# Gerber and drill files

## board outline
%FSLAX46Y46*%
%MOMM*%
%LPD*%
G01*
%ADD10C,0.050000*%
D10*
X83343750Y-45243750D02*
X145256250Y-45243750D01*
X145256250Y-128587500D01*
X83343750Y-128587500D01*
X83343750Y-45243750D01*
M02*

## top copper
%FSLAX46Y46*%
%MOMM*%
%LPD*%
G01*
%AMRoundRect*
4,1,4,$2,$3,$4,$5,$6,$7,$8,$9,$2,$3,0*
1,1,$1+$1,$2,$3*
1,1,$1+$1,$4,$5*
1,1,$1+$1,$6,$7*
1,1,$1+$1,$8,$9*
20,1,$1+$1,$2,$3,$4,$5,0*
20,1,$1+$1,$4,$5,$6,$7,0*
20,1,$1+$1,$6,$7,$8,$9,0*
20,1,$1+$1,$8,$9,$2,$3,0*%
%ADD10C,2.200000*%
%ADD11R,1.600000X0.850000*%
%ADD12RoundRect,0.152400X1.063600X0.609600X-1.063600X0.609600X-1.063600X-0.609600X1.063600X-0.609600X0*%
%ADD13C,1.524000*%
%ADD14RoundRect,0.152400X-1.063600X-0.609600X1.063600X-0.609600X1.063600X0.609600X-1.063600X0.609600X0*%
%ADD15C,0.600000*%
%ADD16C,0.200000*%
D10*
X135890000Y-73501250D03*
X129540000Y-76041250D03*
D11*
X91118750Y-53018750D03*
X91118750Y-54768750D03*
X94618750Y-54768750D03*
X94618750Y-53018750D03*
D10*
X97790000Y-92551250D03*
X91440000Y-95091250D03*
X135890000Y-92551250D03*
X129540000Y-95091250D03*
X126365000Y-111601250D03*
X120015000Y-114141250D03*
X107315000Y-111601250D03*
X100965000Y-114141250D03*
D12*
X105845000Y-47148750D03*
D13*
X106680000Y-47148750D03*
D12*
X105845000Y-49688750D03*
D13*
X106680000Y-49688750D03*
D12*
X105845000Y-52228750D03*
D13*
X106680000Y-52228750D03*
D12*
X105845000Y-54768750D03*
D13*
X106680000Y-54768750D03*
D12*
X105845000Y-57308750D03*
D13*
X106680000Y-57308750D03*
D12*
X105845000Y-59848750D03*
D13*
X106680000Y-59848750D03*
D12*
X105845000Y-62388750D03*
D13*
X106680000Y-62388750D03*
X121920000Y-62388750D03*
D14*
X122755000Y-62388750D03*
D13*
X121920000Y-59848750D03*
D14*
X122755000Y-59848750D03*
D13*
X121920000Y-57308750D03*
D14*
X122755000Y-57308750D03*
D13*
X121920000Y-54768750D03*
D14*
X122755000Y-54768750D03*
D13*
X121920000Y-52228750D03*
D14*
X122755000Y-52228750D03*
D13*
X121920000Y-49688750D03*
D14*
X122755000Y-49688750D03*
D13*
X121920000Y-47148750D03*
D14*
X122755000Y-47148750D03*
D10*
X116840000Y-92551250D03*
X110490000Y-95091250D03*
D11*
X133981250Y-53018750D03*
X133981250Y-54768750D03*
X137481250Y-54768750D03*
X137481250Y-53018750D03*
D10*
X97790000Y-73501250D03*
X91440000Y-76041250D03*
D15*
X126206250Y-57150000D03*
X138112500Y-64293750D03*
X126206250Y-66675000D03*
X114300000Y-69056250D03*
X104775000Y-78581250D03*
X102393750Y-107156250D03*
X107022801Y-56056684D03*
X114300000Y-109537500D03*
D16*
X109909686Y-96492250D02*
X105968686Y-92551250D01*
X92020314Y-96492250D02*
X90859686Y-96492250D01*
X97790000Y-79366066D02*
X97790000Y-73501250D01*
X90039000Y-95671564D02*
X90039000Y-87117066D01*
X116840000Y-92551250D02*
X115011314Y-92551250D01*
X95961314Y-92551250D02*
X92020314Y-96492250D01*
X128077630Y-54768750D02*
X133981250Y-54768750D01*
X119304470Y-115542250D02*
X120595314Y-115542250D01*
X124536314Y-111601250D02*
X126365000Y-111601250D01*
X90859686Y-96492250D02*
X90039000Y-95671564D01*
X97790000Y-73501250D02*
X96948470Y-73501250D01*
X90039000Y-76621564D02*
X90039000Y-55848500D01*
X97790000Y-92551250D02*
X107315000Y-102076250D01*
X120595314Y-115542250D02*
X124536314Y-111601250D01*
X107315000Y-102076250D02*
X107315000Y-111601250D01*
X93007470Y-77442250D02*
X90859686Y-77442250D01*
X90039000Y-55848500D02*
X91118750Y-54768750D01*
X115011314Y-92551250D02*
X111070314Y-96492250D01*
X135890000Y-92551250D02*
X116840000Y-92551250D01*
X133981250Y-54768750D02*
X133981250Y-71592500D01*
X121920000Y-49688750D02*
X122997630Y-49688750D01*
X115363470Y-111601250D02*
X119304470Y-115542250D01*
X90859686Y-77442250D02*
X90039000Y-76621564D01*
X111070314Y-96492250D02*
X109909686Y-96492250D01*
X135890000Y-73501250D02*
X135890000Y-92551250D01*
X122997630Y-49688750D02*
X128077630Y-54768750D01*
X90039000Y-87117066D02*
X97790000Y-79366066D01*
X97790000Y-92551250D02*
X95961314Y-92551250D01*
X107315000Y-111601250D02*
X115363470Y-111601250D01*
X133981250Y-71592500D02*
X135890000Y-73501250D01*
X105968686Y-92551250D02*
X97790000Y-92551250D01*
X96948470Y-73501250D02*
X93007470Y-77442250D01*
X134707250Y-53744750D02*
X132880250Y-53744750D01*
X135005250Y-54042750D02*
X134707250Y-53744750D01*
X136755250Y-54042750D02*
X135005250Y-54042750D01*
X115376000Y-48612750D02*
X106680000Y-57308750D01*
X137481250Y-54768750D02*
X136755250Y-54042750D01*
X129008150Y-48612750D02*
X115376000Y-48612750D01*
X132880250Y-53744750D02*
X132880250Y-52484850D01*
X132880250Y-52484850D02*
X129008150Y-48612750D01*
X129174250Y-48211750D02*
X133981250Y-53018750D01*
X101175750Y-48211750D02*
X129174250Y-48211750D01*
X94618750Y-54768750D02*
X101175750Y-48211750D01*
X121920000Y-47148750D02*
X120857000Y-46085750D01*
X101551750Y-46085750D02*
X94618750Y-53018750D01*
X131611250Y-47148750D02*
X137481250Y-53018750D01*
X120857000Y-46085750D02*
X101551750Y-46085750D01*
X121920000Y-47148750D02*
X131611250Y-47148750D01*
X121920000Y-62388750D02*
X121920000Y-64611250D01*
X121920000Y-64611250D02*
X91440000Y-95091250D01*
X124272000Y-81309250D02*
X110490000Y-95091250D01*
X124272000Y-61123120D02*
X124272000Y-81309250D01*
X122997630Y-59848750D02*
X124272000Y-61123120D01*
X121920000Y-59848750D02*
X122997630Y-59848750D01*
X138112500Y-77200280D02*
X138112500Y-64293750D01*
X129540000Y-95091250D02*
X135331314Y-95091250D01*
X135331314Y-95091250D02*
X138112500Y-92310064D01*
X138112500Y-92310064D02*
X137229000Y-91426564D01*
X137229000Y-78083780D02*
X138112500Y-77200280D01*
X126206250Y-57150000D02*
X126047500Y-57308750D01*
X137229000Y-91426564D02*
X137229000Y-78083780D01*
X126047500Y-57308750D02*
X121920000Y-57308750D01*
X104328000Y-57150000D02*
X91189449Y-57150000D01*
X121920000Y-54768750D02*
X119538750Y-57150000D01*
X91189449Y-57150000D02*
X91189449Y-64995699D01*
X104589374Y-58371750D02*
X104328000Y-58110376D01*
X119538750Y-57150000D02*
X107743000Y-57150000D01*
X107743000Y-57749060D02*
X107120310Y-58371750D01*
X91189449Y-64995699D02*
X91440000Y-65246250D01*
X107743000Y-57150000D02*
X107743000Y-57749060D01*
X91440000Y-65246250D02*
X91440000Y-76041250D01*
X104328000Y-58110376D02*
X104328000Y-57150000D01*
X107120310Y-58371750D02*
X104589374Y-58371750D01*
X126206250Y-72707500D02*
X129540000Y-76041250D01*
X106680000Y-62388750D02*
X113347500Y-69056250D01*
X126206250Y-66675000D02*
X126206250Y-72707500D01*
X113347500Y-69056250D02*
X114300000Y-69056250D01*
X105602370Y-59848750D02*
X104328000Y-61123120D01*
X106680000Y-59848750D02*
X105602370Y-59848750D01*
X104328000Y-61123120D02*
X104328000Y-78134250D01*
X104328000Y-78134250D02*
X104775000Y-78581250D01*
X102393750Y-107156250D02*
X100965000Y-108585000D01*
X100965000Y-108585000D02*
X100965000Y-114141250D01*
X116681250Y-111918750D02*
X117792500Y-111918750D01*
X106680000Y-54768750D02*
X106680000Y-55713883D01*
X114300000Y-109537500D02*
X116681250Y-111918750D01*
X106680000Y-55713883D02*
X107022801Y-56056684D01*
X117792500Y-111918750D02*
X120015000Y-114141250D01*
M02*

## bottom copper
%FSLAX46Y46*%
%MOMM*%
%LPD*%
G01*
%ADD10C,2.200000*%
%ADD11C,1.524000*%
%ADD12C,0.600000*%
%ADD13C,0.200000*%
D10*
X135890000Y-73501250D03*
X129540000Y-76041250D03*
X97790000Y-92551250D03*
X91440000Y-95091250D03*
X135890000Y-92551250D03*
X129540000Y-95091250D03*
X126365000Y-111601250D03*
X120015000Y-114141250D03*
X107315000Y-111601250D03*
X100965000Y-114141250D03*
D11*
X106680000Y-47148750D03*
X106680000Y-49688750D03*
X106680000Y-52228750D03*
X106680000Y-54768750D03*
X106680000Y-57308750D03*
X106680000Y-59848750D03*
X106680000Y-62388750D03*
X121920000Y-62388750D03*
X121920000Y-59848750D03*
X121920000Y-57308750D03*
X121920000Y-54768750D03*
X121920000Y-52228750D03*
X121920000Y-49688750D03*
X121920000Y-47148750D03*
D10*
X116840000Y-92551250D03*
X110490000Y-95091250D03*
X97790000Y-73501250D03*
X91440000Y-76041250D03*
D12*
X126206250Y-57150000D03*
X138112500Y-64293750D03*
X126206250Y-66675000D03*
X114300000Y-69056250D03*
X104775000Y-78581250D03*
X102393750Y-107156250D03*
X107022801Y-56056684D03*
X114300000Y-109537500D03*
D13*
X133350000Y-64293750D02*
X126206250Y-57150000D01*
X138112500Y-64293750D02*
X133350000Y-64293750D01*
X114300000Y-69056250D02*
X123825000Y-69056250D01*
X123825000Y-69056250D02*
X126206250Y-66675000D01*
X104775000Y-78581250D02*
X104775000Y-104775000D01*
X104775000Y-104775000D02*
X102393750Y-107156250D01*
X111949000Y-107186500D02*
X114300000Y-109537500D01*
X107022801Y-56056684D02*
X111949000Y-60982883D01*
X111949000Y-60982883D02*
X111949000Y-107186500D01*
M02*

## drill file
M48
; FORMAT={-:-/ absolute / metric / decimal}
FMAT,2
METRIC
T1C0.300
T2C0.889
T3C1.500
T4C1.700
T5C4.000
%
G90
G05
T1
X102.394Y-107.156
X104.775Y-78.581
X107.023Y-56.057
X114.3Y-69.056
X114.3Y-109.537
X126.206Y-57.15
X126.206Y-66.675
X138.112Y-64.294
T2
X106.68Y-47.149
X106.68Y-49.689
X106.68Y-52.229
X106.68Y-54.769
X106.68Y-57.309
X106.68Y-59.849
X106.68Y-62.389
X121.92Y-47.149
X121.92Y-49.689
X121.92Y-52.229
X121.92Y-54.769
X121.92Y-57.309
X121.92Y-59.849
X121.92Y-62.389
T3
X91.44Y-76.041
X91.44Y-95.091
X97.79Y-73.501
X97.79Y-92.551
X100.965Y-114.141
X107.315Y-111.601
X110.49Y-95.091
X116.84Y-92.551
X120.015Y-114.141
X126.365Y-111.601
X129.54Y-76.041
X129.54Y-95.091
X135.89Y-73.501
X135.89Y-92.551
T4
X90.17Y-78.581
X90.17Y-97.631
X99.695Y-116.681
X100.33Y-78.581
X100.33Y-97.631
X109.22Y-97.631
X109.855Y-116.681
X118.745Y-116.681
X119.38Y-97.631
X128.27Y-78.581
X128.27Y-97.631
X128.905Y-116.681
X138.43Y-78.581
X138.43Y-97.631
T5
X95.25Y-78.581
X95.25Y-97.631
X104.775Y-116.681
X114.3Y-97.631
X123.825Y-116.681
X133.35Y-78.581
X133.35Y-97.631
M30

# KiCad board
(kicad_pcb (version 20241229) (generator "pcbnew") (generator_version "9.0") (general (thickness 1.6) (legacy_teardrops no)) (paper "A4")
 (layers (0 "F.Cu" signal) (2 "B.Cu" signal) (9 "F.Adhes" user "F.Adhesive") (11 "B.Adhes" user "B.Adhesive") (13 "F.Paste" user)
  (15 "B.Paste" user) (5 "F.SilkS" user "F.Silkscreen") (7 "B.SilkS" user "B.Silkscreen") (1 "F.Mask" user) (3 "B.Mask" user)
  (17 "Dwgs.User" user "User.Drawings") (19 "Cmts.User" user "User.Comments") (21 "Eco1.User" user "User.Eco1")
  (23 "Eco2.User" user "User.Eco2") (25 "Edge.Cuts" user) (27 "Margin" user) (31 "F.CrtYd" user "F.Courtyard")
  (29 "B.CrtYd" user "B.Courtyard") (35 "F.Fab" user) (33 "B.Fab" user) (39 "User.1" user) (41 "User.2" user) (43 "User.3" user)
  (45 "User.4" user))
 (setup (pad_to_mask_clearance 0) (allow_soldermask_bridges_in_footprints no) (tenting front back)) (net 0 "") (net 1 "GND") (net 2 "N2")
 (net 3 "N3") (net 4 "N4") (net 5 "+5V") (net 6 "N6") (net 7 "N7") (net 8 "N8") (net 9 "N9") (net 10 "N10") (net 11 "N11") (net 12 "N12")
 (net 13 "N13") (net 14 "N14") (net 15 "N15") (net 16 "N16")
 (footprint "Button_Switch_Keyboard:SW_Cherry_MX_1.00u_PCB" (layer "F.Cu") (at 135.89 73.50125)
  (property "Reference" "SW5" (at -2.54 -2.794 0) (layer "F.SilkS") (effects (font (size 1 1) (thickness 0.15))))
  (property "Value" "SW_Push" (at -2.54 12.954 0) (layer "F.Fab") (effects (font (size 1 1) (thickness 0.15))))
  (pad "" np_thru_hole circle (at -7.62 5.08) (size 1.7 1.7) (drill 1.7) (layers "*.Cu" "*.Mask"))
  (pad "" np_thru_hole circle (at -2.54 5.08) (size 4 4) (drill 4) (layers "*.Cu" "*.Mask"))
  (pad "" np_thru_hole circle (at 2.54 5.08) (size 1.7 1.7) (drill 1.7) (layers "*.Cu" "*.Mask"))
  (pad "1" thru_hole circle (at 0 0) (size 2.2 2.2) (drill 1.5) (layers "*.Cu" "*.Mask") (remove_unused_layers no) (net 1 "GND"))
  (pad "2" thru_hole circle (at -6.35 2.54) (size 2.2 2.2) (drill 1.5) (layers "*.Cu" "*.Mask") (remove_unused_layers no) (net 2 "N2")))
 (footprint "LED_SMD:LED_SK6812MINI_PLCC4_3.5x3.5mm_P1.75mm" (layer "F.Cu") (at 92.86875 53.89375)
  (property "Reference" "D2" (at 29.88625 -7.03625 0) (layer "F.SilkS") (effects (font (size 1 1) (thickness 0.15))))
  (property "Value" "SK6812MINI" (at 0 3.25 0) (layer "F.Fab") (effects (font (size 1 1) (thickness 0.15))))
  (pad "1" smd rect (at -1.75 -0.875) (size 1.6 0.85) (layers "F.Cu" "F.Mask" "F.Paste") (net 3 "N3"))
  (pad "2" smd rect (at -1.75 0.875) (size 1.6 0.85) (layers "F.Cu" "F.Mask" "F.Paste") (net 1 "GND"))
  (pad "3" smd rect (at 1.75 0.875) (size 1.6 0.85) (layers "F.Cu" "F.Mask" "F.Paste") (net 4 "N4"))
  (pad "4" smd rect (at 1.75 -0.875) (size 1.6 0.85) (layers "F.Cu" "F.Mask" "F.Paste") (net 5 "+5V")))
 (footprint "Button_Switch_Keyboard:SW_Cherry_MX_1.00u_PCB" (layer "F.Cu") (at 97.79 92.55125)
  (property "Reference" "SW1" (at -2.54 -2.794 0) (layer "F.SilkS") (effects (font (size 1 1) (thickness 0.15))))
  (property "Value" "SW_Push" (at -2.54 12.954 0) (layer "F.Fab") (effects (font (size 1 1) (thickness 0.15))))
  (pad "" np_thru_hole circle (at -7.62 5.08) (size 1.7 1.7) (drill 1.7) (layers "*.Cu" "*.Mask"))
  (pad "" np_thru_hole circle (at -2.54 5.08) (size 4 4) (drill 4) (layers "*.Cu" "*.Mask"))
  (pad "" np_thru_hole circle (at 2.54 5.08) (size 1.7 1.7) (drill 1.7) (layers "*.Cu" "*.Mask"))
  (pad "1" thru_hole circle (at 0 0) (size 2.2 2.2) (drill 1.5) (layers "*.Cu" "*.Mask") (remove_unused_layers no) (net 1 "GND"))
  (pad "2" thru_hole circle (at -6.35 2.54) (size 2.2 2.2) (drill 1.5) (layers "*.Cu" "*.Mask") (remove_unused_layers no) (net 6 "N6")))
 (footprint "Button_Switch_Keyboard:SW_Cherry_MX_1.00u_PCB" (layer "F.Cu") (at 135.89 92.55125)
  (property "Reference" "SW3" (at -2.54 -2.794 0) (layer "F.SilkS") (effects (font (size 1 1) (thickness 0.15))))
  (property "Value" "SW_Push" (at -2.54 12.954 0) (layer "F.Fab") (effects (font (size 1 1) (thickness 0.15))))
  (pad "" np_thru_hole circle (at -7.62 5.08) (size 1.7 1.7) (drill 1.7) (layers "*.Cu" "*.Mask"))
  (pad "" np_thru_hole circle (at -2.54 5.08) (size 4 4) (drill 4) (layers "*.Cu" "*.Mask"))
  (pad "" np_thru_hole circle (at 2.54 5.08) (size 1.7 1.7) (drill 1.7) (layers "*.Cu" "*.Mask"))
  (pad "1" thru_hole circle (at 0 0) (size 2.2 2.2) (drill 1.5) (layers "*.Cu" "*.Mask") (remove_unused_layers no) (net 1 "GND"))
  (pad "2" thru_hole circle (at -6.35 2.54) (size 2.2 2.2) (drill 1.5) (layers "*.Cu" "*.Mask") (remove_unused_layers no) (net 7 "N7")))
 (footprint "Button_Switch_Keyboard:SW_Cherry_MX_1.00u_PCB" (layer "F.Cu") (at 126.365 111.60125)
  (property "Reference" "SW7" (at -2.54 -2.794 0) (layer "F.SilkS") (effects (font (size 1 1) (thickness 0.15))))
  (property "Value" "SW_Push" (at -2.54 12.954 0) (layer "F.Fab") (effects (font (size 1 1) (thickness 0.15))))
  (pad "" np_thru_hole circle (at -7.62 5.08) (size 1.7 1.7) (drill 1.7) (layers "*.Cu" "*.Mask"))
  (pad "" np_thru_hole circle (at -2.54 5.08) (size 4 4) (drill 4) (layers "*.Cu" "*.Mask"))
  (pad "" np_thru_hole circle (at 2.54 5.08) (size 1.7 1.7) (drill 1.7) (layers "*.Cu" "*.Mask"))
  (pad "1" thru_hole circle (at 0 0) (size 2.2 2.2) (drill 1.5) (layers "*.Cu" "*.Mask") (remove_unused_layers no) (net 1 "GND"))
  (pad "2" thru_hole circle (at -6.35 2.54) (size 2.2 2.2) (drill 1.5) (layers "*.Cu" "*.Mask") (remove_unused_layers no) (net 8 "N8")))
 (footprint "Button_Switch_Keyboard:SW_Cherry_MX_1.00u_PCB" (layer "F.Cu") (at 107.315 111.60125)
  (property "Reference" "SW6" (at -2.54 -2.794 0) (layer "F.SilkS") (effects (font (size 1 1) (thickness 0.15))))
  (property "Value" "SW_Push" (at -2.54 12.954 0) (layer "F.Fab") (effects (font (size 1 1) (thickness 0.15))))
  (pad "" np_thru_hole circle (at -7.62 5.08) (size 1.7 1.7) (drill 1.7) (layers "*.Cu" "*.Mask"))
  (pad "" np_thru_hole circle (at -2.54 5.08) (size 4 4) (drill 4) (layers "*.Cu" "*.Mask"))
  (pad "" np_thru_hole circle (at 2.54 5.08) (size 1.7 1.7) (drill 1.7) (layers "*.Cu" "*.Mask"))
  (pad "1" thru_hole circle (at 0 0) (size 2.2 2.2) (drill 1.5) (layers "*.Cu" "*.Mask") (remove_unused_layers no) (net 1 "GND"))
  (pad "2" thru_hole circle (at -6.35 2.54) (size 2.2 2.2) (drill 1.5) (layers "*.Cu" "*.Mask") (remove_unused_layers no) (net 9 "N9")))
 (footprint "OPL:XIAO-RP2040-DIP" (layer "F.Cu") (at 114.3 54.76875)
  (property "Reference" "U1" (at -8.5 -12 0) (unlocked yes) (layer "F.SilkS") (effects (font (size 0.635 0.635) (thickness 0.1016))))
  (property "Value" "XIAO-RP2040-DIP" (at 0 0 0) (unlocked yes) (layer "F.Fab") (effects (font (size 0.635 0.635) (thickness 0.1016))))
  (pad "1" smd roundrect (at -8.455 -7.62 180) (size 2.432 1.524) (layers "F.Cu" "F.Mask") (roundrect_rratio 0.1) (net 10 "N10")
   (thermal_bridge_angle 45))
  (pad "1" thru_hole circle (at -7.62 -7.62 180) (size 1.524 1.524) (drill 0.889) (layers "*.Cu" "*.Mask") (remove_unused_layers no)
   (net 10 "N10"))
  (pad "2" smd roundrect (at -8.455 -5.08 180) (size 2.432 1.524) (layers "F.Cu" "F.Mask") (roundrect_rratio 0.1) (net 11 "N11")
   (thermal_bridge_angle 45))
  (pad "2" thru_hole circle (at -7.62 -5.08 180) (size 1.524 1.524) (drill 0.889) (layers "*.Cu" "*.Mask") (remove_unused_layers no)
   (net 11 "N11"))
  (pad "3" smd roundrect (at -8.455 -2.54 180) (size 2.432 1.524) (layers "F.Cu" "F.Mask") (roundrect_rratio 0.1) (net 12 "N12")
   (thermal_bridge_angle 45))
  (pad "3" thru_hole circle (at -7.62 -2.54 180) (size 1.524 1.524) (drill 0.889) (layers "*.Cu" "*.Mask") (remove_unused_layers no)
   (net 12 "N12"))
  (pad "4" smd roundrect (at -8.455 0 180) (size 2.432 1.524) (layers "F.Cu" "F.Mask") (roundrect_rratio 0.1) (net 8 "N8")
   (thermal_bridge_angle 45))
  (pad "4" thru_hole circle (at -7.62 0 180) (size 1.524 1.524) (drill 0.889) (layers "*.Cu" "*.Mask") (remove_unused_layers no)
   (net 8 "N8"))
  (pad "5" smd roundrect (at -8.455 2.54 180) (size 2.432 1.524) (layers "F.Cu" "F.Mask") (roundrect_rratio 0.1) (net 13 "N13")
   (thermal_bridge_angle 45))
  (pad "5" thru_hole circle (at -7.62 2.54 180) (size 1.524 1.524) (drill 0.889) (layers "*.Cu" "*.Mask") (remove_unused_layers no)
   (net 13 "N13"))
  (pad "6" smd roundrect (at -8.455 5.08 180) (size 2.432 1.524) (layers "F.Cu" "F.Mask") (roundrect_rratio 0.1) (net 9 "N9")
   (thermal_bridge_angle 45))
  (pad "6" thru_hole circle (at -7.62 5.08 180) (size 1.524 1.524) (drill 0.889) (layers "*.Cu" "*.Mask") (remove_unused_layers no)
   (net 9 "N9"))
  (pad "7" smd roundrect (at -8.455 7.62 180) (size 2.432 1.524) (layers "F.Cu" "F.Mask") (roundrect_rratio 0.1) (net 2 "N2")
   (thermal_bridge_angle 45))
  (pad "7" thru_hole circle (at -7.62 7.62 180) (size 1.524 1.524) (drill 0.889) (layers "*.Cu" "*.Mask") (remove_unused_layers no)
   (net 2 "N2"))
  (pad "8" thru_hole circle (at 7.62 7.62) (size 1.524 1.524) (drill 0.889) (layers "*.Cu" "*.Mask") (remove_unused_layers no) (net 6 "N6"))
  (pad "8" smd roundrect (at 8.455 7.62) (size 2.432 1.524) (layers "F.Cu" "F.Mask") (roundrect_rratio 0.1) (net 6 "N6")
   (thermal_bridge_angle 45))
  (pad "9" thru_hole circle (at 7.62 5.08) (size 1.524 1.524) (drill 0.889) (layers "*.Cu" "*.Mask") (remove_unused_layers no)
   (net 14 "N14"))
  (pad "9" smd roundrect (at 8.455 5.08) (size 2.432 1.524) (layers "F.Cu" "F.Mask") (roundrect_rratio 0.1) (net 14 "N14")
   (thermal_bridge_angle 45))
  (pad "10" thru_hole circle (at 7.62 2.54) (size 1.524 1.524) (drill 0.889) (layers "*.Cu" "*.Mask") (remove_unused_layers no) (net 7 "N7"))
  (pad "10" smd roundrect (at 8.455 2.54) (size 2.432 1.524) (layers "F.Cu" "F.Mask") (roundrect_rratio 0.1) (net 7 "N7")
   (thermal_bridge_angle 45))
  (pad "11" thru_hole circle (at 7.62 0) (size 1.524 1.524) (drill 0.889) (layers "*.Cu" "*.Mask") (remove_unused_layers no) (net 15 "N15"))
  (pad "11" smd roundrect (at 8.455 0) (size 2.432 1.524) (layers "F.Cu" "F.Mask") (roundrect_rratio 0.1) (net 15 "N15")
   (thermal_bridge_angle 45))
  (pad "12" thru_hole circle (at 7.62 -2.54) (size 1.524 1.524) (drill 0.889) (layers "*.Cu" "*.Mask") (remove_unused_layers no)
   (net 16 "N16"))
  (pad "12" smd roundrect (at 8.455 -2.54) (size 2.432 1.524) (layers "F.Cu" "F.Mask") (roundrect_rratio 0.1) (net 16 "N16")
   (thermal_bridge_angle 45))
  (pad "13" thru_hole circle (at 7.62 -5.08) (size 1.524 1.524) (drill 0.889) (layers "*.Cu" "*.Mask") (remove_unused_layers no)
   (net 1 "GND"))
  (pad "13" smd roundrect (at 8.455 -5.08) (size 2.432 1.524) (layers "F.Cu" "F.Mask") (roundrect_rratio 0.1) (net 1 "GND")
   (thermal_bridge_angle 45))
  (pad "14" thru_hole circle (at 7.62 -7.62) (size 1.524 1.524) (drill 0.889) (layers "*.Cu" "*.Mask") (remove_unused_layers no)
   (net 5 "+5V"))
  (pad "14" smd roundrect (at 8.455 -7.62) (size 2.432 1.524) (layers "F.Cu" "F.Mask") (roundrect_rratio 0.1) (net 5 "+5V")
   (thermal_bridge_angle 45)))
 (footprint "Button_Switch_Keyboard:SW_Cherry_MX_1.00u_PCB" (layer "F.Cu") (at 116.84 92.55125)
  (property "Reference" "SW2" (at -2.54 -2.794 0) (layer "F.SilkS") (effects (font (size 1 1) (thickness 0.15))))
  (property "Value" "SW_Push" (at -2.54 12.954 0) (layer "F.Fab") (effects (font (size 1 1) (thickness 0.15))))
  (pad "" np_thru_hole circle (at -7.62 5.08) (size 1.7 1.7) (drill 1.7) (layers "*.Cu" "*.Mask"))
  (pad "" np_thru_hole circle (at -2.54 5.08) (size 4 4) (drill 4) (layers "*.Cu" "*.Mask"))
  (pad "" np_thru_hole circle (at 2.54 5.08) (size 1.7 1.7) (drill 1.7) (layers "*.Cu" "*.Mask"))
  (pad "1" thru_hole circle (at 0 0) (size 2.2 2.2) (drill 1.5) (layers "*.Cu" "*.Mask") (remove_unused_layers no) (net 1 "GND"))
  (pad "2" thru_hole circle (at -6.35 2.54) (size 2.2 2.2) (drill 1.5) (layers "*.Cu" "*.Mask") (remove_unused_layers no) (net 14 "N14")))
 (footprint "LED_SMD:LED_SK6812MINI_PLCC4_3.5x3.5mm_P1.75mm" (layer "F.Cu") (at 135.73125 53.89375)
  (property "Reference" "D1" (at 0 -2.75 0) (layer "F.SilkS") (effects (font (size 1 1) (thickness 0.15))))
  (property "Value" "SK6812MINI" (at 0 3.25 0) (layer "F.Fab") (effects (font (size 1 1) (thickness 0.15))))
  (pad "1" smd rect (at -1.75 -0.875) (size 1.6 0.85) (layers "F.Cu" "F.Mask" "F.Paste") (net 4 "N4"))
  (pad "2" smd rect (at -1.75 0.875) (size 1.6 0.85) (layers "F.Cu" "F.Mask" "F.Paste") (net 1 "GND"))
  (pad "3" smd rect (at 1.75 0.875) (size 1.6 0.85) (layers "F.Cu" "F.Mask" "F.Paste") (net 13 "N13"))
  (pad "4" smd rect (at 1.75 -0.875) (size 1.6 0.85) (layers "F.Cu" "F.Mask" "F.Paste") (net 5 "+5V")))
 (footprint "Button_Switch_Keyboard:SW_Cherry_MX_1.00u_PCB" (layer "F.Cu") (at 97.79 73.50125)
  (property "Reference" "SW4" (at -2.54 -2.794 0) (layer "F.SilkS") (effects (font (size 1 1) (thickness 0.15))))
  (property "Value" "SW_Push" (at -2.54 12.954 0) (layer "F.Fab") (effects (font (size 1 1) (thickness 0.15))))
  (pad "" np_thru_hole circle (at -7.62 5.08) (size 1.7 1.7) (drill 1.7) (layers "*.Cu" "*.Mask"))
  (pad "" np_thru_hole circle (at -2.54 5.08) (size 4 4) (drill 4) (layers "*.Cu" "*.Mask"))
  (pad "" np_thru_hole circle (at 2.54 5.08) (size 1.7 1.7) (drill 1.7) (layers "*.Cu" "*.Mask"))
  (pad "1" thru_hole circle (at 0 0) (size 2.2 2.2) (drill 1.5) (layers "*.Cu" "*.Mask") (remove_unused_layers no) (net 1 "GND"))
  (pad "2" thru_hole circle (at -6.35 2.54) (size 2.2 2.2) (drill 1.5) (layers "*.Cu" "*.Mask") (remove_unused_layers no) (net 15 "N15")))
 (gr_rect (start 83.34375 45.24375) (end 145.25625 128.5875) (stroke (width 0.05) (type default)) (fill no) (layer "Edge.Cuts"))
 (segment (start 109.909686 96.49225) (end 105.968686 92.55125) (width 0.2) (layer "F.Cu") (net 1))
 (segment (start 92.020314 96.49225) (end 90.859686 96.49225) (width 0.2) (layer "F.Cu") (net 1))
 (segment (start 97.79 79.366066) (end 97.79 73.50125) (width 0.2) (layer "F.Cu") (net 1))
 (segment (start 90.039 95.671564) (end 90.039 87.117066) (width 0.2) (layer "F.Cu") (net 1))
 (segment (start 116.84 92.55125) (end 115.011314 92.55125) (width 0.2) (layer "F.Cu") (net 1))
 (segment (start 95.961314 92.55125) (end 92.020314 96.49225) (width 0.2) (layer "F.Cu") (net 1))
 (segment (start 128.07763 54.76875) (end 133.98125 54.76875) (width 0.2) (layer "F.Cu") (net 1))
 (segment (start 119.30447 115.54225) (end 120.595314 115.54225) (width 0.2) (layer "F.Cu") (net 1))
 (segment (start 124.536314 111.60125) (end 126.365 111.60125) (width 0.2) (layer "F.Cu") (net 1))
 (segment (start 90.859686 96.49225) (end 90.039 95.671564) (width 0.2) (layer "F.Cu") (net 1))
 (segment (start 97.79 73.50125) (end 96.94847 73.50125) (width 0.2) (layer "F.Cu") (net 1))
 (segment (start 90.039 76.621564) (end 90.039 55.8485) (width 0.2) (layer "F.Cu") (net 1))
 (segment (start 97.79 92.55125) (end 107.315 102.07625) (width 0.2) (layer "F.Cu") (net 1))
 (segment (start 120.595314 115.54225) (end 124.536314 111.60125) (width 0.2) (layer "F.Cu") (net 1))
 (segment (start 107.315 102.07625) (end 107.315 111.60125) (width 0.2) (layer "F.Cu") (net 1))
 (segment (start 93.00747 77.44225) (end 90.859686 77.44225) (width 0.2) (layer "F.Cu") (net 1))
 (segment (start 90.039 55.8485) (end 91.11875 54.76875) (width 0.2) (layer "F.Cu") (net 1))
 (segment (start 115.011314 92.55125) (end 111.070314 96.49225) (width 0.2) (layer "F.Cu") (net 1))
 (segment (start 135.89 92.55125) (end 116.84 92.55125) (width 0.2) (layer "F.Cu") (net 1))
 (segment (start 133.98125 54.76875) (end 133.98125 71.5925) (width 0.2) (layer "F.Cu") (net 1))
 (segment (start 121.92 49.68875) (end 122.99763 49.68875) (width 0.2) (layer "F.Cu") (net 1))
 (segment (start 115.36347 111.60125) (end 119.30447 115.54225) (width 0.2) (layer "F.Cu") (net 1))
 (segment (start 90.859686 77.44225) (end 90.039 76.621564) (width 0.2) (layer "F.Cu") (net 1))
 (segment (start 111.070314 96.49225) (end 109.909686 96.49225) (width 0.2) (layer "F.Cu") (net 1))
 (segment (start 135.89 73.50125) (end 135.89 92.55125) (width 0.2) (layer "F.Cu") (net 1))
 (segment (start 122.99763 49.68875) (end 128.07763 54.76875) (width 0.2) (layer "F.Cu") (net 1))
 (segment (start 90.039 87.117066) (end 97.79 79.366066) (width 0.2) (layer "F.Cu") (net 1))
 (segment (start 97.79 92.55125) (end 95.961314 92.55125) (width 0.2) (layer "F.Cu") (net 1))
 (segment (start 107.315 111.60125) (end 115.36347 111.60125) (width 0.2) (layer "F.Cu") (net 1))
 (segment (start 133.98125 71.5925) (end 135.89 73.50125) (width 0.2) (layer "F.Cu") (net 1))
 (segment (start 105.968686 92.55125) (end 97.79 92.55125) (width 0.2) (layer "F.Cu") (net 1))
 (segment (start 96.94847 73.50125) (end 93.00747 77.44225) (width 0.2) (layer "F.Cu") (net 1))
 (segment (start 134.70725 53.74475) (end 132.88025 53.74475) (width 0.2) (layer "F.Cu") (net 13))
 (segment (start 135.00525 54.04275) (end 134.70725 53.74475) (width 0.2) (layer "F.Cu") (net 13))
 (segment (start 136.75525 54.04275) (end 135.00525 54.04275) (width 0.2) (layer "F.Cu") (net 13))
 (segment (start 115.376 48.61275) (end 106.68 57.30875) (width 0.2) (layer "F.Cu") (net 13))
 (segment (start 137.48125 54.76875) (end 136.75525 54.04275) (width 0.2) (layer "F.Cu") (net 13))
 (segment (start 129.00815 48.61275) (end 115.376 48.61275) (width 0.2) (layer "F.Cu") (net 13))
 (segment (start 132.88025 53.74475) (end 132.88025 52.48485) (width 0.2) (layer "F.Cu") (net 13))
 (segment (start 132.88025 52.48485) (end 129.00815 48.61275) (width 0.2) (layer "F.Cu") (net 13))
 (segment (start 129.17425 48.21175) (end 133.98125 53.01875) (width 0.2) (layer "F.Cu") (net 4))
 (segment (start 101.17575 48.21175) (end 129.17425 48.21175) (width 0.2) (layer "F.Cu") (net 4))
 (segment (start 94.61875 54.76875) (end 101.17575 48.21175) (width 0.2) (layer "F.Cu") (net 4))
 (segment (start 121.92 47.14875) (end 120.857 46.08575) (width 0.2) (layer "F.Cu") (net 5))
 (segment (start 101.55175 46.08575) (end 94.61875 53.01875) (width 0.2) (layer "F.Cu") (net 5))
 (segment (start 131.61125 47.14875) (end 137.48125 53.01875) (width 0.2) (layer "F.Cu") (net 5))
 (segment (start 120.857 46.08575) (end 101.55175 46.08575) (width 0.2) (layer "F.Cu") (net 5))
 (segment (start 121.92 47.14875) (end 131.61125 47.14875) (width 0.2) (layer "F.Cu") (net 5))
 (segment (start 121.92 62.38875) (end 121.92 64.61125) (width 0.2) (layer "F.Cu") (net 6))
 (segment (start 121.92 64.61125) (end 91.44 95.09125) (width 0.2) (layer "F.Cu") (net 6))
 (segment (start 124.272 81.30925) (end 110.49 95.09125) (width 0.2) (layer "F.Cu") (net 14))
 (segment (start 124.272 61.12312) (end 124.272 81.30925) (width 0.2) (layer "F.Cu") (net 14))
 (segment (start 122.99763 59.84875) (end 124.272 61.12312) (width 0.2) (layer "F.Cu") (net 14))
 (segment (start 121.92 59.84875) (end 122.99763 59.84875) (width 0.2) (layer "F.Cu") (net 14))
 (segment (start 138.1125 77.20028) (end 138.1125 64.29375) (width 0.2) (layer "F.Cu") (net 7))
 (segment (start 129.54 95.09125) (end 135.331314 95.09125) (width 0.2) (layer "F.Cu") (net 7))
 (segment (start 135.331314 95.09125) (end 138.1125 92.310064) (width 0.2) (layer "F.Cu") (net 7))
 (segment (start 138.1125 92.310064) (end 137.229 91.426564) (width 0.2) (layer "F.Cu") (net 7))
 (segment (start 137.229 78.08378) (end 138.1125 77.20028) (width 0.2) (layer "F.Cu") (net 7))
 (segment (start 126.20625 57.15) (end 126.0475 57.30875) (width 0.2) (layer "F.Cu") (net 7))
 (segment (start 137.229 91.426564) (end 137.229 78.08378) (width 0.2) (layer "F.Cu") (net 7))
 (segment (start 126.0475 57.30875) (end 121.92 57.30875) (width 0.2) (layer "F.Cu") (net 7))
 (via (at 126.20625 57.15) (size 0.6) (drill 0.3) (layers "F.Cu" "B.Cu") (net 7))
 (via (at 138.1125 64.29375) (size 0.6) (drill 0.3) (layers "F.Cu" "B.Cu") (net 7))
 (segment (start 133.35 64.29375) (end 126.20625 57.15) (width 0.2) (layer "B.Cu") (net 7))
 (segment (start 138.1125 64.29375) (end 133.35 64.29375) (width 0.2) (layer "B.Cu") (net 7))
 (segment (start 104.328 57.15) (end 91.189449 57.15) (width 0.2) (layer "F.Cu") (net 15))
 (segment (start 121.92 54.76875) (end 119.53875 57.15) (width 0.2) (layer "F.Cu") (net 15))
 (segment (start 91.189449 57.15) (end 91.189449 64.995699) (width 0.2) (layer "F.Cu") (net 15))
 (segment (start 104.589374 58.37175) (end 104.328 58.110376) (width 0.2) (layer "F.Cu") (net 15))
 (segment (start 119.53875 57.15) (end 107.743 57.15) (width 0.2) (layer "F.Cu") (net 15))
 (segment (start 107.743 57.74906) (end 107.12031 58.37175) (width 0.2) (layer "F.Cu") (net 15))
 (segment (start 91.189449 64.995699) (end 91.44 65.24625) (width 0.2) (layer "F.Cu") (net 15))
 (segment (start 107.743 57.15) (end 107.743 57.74906) (width 0.2) (layer "F.Cu") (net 15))
 (segment (start 91.44 65.24625) (end 91.44 76.04125) (width 0.2) (layer "F.Cu") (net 15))
 (segment (start 104.328 58.110376) (end 104.328 57.15) (width 0.2) (layer "F.Cu") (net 15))
 (segment (start 107.12031 58.37175) (end 104.589374 58.37175) (width 0.2) (layer "F.Cu") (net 15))
 (segment (start 126.20625 72.7075) (end 129.54 76.04125) (width 0.2) (layer "F.Cu") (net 2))
 (segment (start 106.68 62.38875) (end 113.3475 69.05625) (width 0.2) (layer "F.Cu") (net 2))
 (segment (start 126.20625 66.675) (end 126.20625 72.7075) (width 0.2) (layer "F.Cu") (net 2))
 (segment (start 113.3475 69.05625) (end 114.3 69.05625) (width 0.2) (layer "F.Cu") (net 2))
 (via (at 126.20625 66.675) (size 0.6) (drill 0.3) (layers "F.Cu" "B.Cu") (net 2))
 (via (at 114.3 69.05625) (size 0.6) (drill 0.3) (layers "F.Cu" "B.Cu") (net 2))
 (segment (start 114.3 69.05625) (end 123.825 69.05625) (width 0.2) (layer "B.Cu") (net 2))
 (segment (start 123.825 69.05625) (end 126.20625 66.675) (width 0.2) (layer "B.Cu") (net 2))
 (segment (start 105.60237 59.84875) (end 104.328 61.12312) (width 0.2) (layer "F.Cu") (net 9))
 (segment (start 106.68 59.84875) (end 105.60237 59.84875) (width 0.2) (layer "F.Cu") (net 9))
 (segment (start 104.328 61.12312) (end 104.328 78.13425) (width 0.2) (layer "F.Cu") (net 9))
 (segment (start 104.328 78.13425) (end 104.775 78.58125) (width 0.2) (layer "F.Cu") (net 9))
 (segment (start 102.39375 107.15625) (end 100.965 108.585) (width 0.2) (layer "F.Cu") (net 9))
 (segment (start 100.965 108.585) (end 100.965 114.14125) (width 0.2) (layer "F.Cu") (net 9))
 (via (at 104.775 78.58125) (size 0.6) (drill 0.3) (layers "F.Cu" "B.Cu") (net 9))
 (via (at 102.39375 107.15625) (size 0.6) (drill 0.3) (layers "F.Cu" "B.Cu") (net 9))
 (segment (start 104.775 78.58125) (end 104.775 104.775) (width 0.2) (layer "B.Cu") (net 9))
 (segment (start 104.775 104.775) (end 102.39375 107.15625) (width 0.2) (layer "B.Cu") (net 9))
 (segment (start 116.68125 111.91875) (end 117.7925 111.91875) (width 0.2) (layer "F.Cu") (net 8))
 (segment (start 106.68 54.76875) (end 106.68 55.713883) (width 0.2) (layer "F.Cu") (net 8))
 (segment (start 114.3 109.5375) (end 116.68125 111.91875) (width 0.2) (layer "F.Cu") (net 8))
 (segment (start 106.68 55.713883) (end 107.022801 56.056684) (width 0.2) (layer "F.Cu") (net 8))
 (segment (start 117.7925 111.91875) (end 120.015 114.14125) (width 0.2) (layer "F.Cu") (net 8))
 (via (at 107.022801 56.056684) (size 0.6) (drill 0.3) (layers "F.Cu" "B.Cu") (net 8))
 (via (at 114.3 109.5375) (size 0.6) (drill 0.3) (layers "F.Cu" "B.Cu") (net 8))
 (segment (start 111.949 107.1865) (end 114.3 109.5375) (width 0.2) (layer "B.Cu") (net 8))
 (segment (start 107.022801 56.056684) (end 111.949 60.982883) (width 0.2) (layer "B.Cu") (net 8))
 (segment (start 111.949 60.982883) (end 111.949 107.1865) (width 0.2) (layer "B.Cu") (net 8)))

